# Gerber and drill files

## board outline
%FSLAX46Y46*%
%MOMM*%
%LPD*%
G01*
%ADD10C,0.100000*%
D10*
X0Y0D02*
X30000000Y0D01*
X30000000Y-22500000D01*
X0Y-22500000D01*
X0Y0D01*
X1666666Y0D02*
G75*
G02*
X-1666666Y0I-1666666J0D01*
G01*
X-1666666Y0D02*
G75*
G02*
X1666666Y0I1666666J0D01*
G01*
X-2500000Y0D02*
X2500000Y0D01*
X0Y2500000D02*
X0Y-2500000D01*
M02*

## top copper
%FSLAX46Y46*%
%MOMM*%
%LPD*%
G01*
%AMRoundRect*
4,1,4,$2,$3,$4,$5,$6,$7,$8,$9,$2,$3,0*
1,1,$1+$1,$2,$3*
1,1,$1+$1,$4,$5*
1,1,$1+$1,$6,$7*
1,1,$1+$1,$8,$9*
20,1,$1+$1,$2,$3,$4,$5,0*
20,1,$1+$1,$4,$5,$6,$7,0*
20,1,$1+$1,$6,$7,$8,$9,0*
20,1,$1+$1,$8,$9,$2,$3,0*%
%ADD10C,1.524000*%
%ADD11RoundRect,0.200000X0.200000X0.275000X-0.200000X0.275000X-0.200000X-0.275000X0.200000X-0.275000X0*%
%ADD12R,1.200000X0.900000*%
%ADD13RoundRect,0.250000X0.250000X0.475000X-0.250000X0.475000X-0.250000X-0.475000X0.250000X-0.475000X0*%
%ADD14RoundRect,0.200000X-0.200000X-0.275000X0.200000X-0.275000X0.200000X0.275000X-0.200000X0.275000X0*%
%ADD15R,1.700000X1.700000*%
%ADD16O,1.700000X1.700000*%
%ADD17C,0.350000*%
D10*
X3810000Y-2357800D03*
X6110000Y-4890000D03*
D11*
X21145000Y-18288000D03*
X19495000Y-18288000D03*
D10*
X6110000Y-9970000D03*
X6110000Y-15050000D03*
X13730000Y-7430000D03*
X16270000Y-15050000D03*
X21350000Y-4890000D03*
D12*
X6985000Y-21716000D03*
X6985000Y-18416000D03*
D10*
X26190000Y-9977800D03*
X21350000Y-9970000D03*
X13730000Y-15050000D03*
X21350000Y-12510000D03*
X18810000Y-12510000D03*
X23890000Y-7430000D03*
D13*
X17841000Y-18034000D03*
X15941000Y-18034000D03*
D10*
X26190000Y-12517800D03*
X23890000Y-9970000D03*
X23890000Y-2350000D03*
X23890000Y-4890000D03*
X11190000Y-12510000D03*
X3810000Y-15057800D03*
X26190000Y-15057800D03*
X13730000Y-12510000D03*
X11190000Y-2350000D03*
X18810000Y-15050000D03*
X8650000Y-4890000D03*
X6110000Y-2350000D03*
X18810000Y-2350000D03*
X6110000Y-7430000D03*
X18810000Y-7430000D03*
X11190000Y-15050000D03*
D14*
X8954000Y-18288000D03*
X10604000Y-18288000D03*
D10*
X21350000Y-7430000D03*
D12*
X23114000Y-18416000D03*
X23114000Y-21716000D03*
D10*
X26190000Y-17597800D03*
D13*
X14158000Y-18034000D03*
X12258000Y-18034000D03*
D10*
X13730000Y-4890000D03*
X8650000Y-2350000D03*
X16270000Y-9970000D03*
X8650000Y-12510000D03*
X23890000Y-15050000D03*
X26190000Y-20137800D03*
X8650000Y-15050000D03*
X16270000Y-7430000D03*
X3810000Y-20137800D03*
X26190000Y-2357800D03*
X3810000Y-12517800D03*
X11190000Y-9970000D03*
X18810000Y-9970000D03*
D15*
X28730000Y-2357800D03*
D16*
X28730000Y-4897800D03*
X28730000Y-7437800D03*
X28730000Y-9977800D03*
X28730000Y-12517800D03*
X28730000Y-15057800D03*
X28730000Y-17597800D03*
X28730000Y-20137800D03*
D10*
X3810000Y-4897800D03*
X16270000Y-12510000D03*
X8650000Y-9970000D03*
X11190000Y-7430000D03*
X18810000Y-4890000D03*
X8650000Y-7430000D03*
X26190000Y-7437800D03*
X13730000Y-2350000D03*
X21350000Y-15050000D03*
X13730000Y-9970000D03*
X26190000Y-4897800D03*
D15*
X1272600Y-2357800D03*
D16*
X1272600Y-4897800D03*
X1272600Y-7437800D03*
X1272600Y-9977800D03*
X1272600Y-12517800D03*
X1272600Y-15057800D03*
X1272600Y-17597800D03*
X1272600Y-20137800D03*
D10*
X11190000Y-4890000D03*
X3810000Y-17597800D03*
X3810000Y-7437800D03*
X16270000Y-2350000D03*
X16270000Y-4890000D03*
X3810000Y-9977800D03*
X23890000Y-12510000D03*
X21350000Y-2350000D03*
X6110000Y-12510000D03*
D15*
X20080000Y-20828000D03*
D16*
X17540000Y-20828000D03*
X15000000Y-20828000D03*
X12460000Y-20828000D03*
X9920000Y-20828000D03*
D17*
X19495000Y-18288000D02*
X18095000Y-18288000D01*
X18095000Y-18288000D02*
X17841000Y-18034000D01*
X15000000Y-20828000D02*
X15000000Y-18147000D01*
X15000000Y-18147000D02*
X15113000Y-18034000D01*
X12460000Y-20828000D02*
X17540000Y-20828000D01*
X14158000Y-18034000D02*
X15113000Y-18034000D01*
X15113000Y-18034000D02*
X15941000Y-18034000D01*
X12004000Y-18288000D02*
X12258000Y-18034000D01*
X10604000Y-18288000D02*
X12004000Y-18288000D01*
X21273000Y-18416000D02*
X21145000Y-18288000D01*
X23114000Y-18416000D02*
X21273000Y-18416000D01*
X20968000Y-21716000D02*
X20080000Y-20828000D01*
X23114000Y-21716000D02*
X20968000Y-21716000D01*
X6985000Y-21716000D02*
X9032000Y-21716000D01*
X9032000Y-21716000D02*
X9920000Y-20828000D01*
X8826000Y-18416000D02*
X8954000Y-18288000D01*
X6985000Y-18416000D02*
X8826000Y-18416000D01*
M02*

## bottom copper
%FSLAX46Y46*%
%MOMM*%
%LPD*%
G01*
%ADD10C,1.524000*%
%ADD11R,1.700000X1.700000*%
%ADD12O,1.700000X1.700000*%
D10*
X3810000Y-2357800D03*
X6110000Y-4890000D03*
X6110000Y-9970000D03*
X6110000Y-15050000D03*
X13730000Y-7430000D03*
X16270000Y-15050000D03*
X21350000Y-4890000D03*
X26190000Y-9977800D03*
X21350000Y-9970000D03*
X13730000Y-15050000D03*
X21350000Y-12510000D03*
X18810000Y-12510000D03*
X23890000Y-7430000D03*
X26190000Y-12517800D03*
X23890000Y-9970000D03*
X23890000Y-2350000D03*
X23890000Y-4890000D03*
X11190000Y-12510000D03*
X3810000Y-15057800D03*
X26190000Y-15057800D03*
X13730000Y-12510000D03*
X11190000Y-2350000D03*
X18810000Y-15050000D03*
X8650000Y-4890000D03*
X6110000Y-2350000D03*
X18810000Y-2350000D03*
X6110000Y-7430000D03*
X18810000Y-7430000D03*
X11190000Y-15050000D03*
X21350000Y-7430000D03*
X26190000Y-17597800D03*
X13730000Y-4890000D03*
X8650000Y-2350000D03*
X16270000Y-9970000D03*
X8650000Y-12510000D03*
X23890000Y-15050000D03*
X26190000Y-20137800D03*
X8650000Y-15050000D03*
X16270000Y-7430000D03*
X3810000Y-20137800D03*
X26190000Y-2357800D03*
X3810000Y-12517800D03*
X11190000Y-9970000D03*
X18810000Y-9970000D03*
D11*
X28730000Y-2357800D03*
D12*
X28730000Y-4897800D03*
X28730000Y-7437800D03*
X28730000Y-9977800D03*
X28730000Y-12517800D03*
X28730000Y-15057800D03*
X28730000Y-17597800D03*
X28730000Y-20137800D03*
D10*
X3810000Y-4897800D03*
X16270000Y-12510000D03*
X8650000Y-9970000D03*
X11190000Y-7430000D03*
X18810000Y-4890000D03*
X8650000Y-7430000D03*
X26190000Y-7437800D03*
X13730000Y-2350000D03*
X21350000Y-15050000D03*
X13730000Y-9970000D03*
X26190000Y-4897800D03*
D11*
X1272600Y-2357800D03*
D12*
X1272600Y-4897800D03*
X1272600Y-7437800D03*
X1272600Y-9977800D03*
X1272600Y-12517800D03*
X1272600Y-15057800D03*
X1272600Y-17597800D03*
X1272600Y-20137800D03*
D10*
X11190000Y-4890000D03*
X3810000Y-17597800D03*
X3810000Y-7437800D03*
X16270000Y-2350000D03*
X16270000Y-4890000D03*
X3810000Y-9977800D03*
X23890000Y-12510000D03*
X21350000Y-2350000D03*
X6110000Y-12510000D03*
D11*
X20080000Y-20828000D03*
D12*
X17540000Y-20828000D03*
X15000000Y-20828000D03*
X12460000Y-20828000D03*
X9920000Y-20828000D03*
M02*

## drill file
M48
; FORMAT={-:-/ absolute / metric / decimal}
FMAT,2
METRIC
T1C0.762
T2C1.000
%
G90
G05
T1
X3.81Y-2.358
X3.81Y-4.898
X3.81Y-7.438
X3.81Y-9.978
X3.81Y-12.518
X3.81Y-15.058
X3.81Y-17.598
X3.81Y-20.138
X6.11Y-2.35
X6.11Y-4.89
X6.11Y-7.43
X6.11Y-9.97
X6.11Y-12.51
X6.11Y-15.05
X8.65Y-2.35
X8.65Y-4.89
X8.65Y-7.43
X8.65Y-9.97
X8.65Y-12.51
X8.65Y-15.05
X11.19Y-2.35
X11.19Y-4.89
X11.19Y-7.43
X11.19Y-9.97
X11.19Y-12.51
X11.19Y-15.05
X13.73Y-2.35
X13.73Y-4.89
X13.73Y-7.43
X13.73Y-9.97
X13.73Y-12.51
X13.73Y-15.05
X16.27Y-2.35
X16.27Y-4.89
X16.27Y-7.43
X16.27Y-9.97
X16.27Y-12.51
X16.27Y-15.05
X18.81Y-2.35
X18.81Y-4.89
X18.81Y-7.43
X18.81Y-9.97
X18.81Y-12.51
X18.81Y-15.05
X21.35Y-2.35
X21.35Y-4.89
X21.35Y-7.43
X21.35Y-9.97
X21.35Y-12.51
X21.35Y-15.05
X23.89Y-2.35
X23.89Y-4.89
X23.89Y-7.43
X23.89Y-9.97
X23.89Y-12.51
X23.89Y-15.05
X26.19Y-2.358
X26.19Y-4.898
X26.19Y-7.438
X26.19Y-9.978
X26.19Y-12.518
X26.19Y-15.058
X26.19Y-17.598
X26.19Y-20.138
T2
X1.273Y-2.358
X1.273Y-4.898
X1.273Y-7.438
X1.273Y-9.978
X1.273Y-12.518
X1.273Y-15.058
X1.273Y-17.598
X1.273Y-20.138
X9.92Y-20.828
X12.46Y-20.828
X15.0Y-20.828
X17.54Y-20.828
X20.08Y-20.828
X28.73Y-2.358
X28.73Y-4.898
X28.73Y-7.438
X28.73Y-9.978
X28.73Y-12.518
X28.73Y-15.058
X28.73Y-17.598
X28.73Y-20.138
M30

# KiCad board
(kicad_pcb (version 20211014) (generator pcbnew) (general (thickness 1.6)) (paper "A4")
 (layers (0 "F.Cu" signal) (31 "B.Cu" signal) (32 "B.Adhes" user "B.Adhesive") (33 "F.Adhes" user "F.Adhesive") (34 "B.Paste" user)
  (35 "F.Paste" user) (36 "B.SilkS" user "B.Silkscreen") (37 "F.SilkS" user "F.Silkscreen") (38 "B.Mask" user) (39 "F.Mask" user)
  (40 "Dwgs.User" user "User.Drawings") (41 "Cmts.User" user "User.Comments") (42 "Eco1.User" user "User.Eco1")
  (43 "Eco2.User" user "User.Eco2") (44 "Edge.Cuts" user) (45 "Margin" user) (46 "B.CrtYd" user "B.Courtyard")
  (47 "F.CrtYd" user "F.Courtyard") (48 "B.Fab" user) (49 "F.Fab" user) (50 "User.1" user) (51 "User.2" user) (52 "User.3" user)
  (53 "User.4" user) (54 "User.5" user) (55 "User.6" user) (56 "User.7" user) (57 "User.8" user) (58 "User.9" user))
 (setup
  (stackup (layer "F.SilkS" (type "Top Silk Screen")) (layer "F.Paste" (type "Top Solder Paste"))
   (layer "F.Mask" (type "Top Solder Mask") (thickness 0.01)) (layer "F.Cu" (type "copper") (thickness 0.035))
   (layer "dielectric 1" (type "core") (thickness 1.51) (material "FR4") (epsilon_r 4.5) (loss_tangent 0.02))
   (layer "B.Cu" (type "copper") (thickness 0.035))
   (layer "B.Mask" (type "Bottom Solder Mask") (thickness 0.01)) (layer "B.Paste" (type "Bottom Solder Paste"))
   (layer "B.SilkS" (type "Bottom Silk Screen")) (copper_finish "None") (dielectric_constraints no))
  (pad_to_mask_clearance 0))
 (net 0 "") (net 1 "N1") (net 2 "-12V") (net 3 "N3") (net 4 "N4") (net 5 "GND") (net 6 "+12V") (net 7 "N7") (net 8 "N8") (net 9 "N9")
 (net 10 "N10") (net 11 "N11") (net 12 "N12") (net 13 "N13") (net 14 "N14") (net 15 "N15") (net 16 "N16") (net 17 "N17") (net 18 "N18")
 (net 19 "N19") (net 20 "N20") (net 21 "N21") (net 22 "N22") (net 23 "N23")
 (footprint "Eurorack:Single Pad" (layer "F.Cu") (at 39.75 2.3578)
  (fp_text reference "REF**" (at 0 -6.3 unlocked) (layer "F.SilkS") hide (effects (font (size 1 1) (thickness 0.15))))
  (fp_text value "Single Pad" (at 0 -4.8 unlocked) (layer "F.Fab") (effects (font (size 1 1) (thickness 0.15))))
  (pad "1" thru_hole circle (at -35.94 0) (size 1.524 1.524) (drill 0.762) (layers *.Cu *.Mask)))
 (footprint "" (layer "F.Cu") (at 6.11 4.89)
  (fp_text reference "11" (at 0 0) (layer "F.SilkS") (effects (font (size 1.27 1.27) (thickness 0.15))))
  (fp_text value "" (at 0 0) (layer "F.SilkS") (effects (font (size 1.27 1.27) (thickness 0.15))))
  (pad "1" thru_hole circle (at 0 0) (size 1.524 1.524) (drill 0.762) (layers *.Cu *.Mask)))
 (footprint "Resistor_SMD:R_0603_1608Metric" (layer "F.Cu") (at 20.32 18.288 180)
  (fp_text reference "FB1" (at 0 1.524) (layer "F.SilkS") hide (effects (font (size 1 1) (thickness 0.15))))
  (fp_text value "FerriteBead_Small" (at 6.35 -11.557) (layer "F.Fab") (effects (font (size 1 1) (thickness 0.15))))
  (pad "1" smd roundrect (at -0.825 0 180) (size 0.8 0.95) (layers "F.Cu" "F.Paste" "F.Mask") (roundrect_rratio 0.25) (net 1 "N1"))
  (pad "2" smd roundrect (at 0.825 0 180) (size 0.8 0.95) (layers "F.Cu" "F.Paste" "F.Mask") (roundrect_rratio 0.25) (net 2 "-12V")))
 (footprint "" (layer "F.Cu") (at 6.11 9.97)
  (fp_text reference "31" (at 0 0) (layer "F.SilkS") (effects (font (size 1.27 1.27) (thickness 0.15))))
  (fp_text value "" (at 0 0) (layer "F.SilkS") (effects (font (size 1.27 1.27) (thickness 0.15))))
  (pad "1" thru_hole circle (at 0 0) (size 1.524 1.524) (drill 0.762) (layers *.Cu *.Mask)))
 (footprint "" (layer "F.Cu") (at 6.11 15.05)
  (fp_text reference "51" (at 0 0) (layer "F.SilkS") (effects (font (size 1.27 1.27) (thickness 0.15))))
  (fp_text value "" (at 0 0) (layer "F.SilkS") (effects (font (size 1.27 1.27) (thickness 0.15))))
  (pad "1" thru_hole circle (at 0 0) (size 1.524 1.524) (drill 0.762) (layers *.Cu *.Mask)))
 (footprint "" (layer "F.Cu") (at 13.73 7.43)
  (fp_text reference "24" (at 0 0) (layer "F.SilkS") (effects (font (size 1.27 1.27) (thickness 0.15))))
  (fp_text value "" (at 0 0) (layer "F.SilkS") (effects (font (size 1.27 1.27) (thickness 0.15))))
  (pad "1" thru_hole circle (at 0 0) (size 1.524 1.524) (drill 0.762) (layers *.Cu *.Mask)))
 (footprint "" (layer "F.Cu") (at 16.27 15.05)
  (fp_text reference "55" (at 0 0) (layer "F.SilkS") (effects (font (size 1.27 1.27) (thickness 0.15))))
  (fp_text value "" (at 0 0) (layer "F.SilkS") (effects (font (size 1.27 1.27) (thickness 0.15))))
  (pad "1" thru_hole circle (at 0 0) (size 1.524 1.524) (drill 0.762) (layers *.Cu *.Mask)))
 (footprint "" (layer "F.Cu") (at 21.35 4.89)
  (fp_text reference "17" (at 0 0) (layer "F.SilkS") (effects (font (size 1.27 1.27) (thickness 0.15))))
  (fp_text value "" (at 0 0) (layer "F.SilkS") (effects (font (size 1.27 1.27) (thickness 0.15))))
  (pad "1" thru_hole circle (at 0 0) (size 1.524 1.524) (drill 0.762) (layers *.Cu *.Mask)))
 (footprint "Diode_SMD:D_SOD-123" (layer "F.Cu") (at 6.985 20.066 90)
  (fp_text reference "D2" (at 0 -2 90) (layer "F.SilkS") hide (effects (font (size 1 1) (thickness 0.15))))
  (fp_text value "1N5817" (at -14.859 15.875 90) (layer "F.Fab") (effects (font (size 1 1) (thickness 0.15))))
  (pad "1" smd rect (at -1.65 0 90) (size 0.9 1.2) (layers "F.Cu" "F.Paste" "F.Mask") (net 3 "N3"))
  (pad "2" smd rect (at 1.65 0 90) (size 0.9 1.2) (layers "F.Cu" "F.Paste" "F.Mask") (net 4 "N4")))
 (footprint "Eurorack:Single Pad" (layer "F.Cu") (at 61.94 9.9778)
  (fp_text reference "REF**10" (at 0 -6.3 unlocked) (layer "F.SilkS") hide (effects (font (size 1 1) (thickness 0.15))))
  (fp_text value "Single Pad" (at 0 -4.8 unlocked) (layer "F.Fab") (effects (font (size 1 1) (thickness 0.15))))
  (pad "1" thru_hole circle (at -35.75 0) (size 1.524 1.524) (drill 0.762) (layers *.Cu *.Mask)))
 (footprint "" (layer "F.Cu") (at 21.35 9.97)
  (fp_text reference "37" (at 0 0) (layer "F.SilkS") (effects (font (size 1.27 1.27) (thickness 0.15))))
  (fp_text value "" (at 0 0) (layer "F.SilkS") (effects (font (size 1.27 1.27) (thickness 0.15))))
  (pad "1" thru_hole circle (at 0 0) (size 1.524 1.524) (drill 0.762) (layers *.Cu *.Mask)))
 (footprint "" (layer "F.Cu") (at 13.73 15.05)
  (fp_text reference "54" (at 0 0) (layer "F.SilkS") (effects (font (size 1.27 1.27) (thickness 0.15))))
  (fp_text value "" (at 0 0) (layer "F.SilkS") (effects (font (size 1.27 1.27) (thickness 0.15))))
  (pad "1" thru_hole circle (at 0 0) (size 1.524 1.524) (drill 0.762) (layers *.Cu *.Mask)))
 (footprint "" (layer "F.Cu") (at 21.35 12.51)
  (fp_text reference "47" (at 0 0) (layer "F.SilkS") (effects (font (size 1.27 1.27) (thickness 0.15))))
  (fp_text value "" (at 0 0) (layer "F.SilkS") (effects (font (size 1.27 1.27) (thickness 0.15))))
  (pad "1" thru_hole circle (at 0 0) (size 1.524 1.524) (drill 0.762) (layers *.Cu *.Mask)))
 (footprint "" (layer "F.Cu") (at 18.81 12.51)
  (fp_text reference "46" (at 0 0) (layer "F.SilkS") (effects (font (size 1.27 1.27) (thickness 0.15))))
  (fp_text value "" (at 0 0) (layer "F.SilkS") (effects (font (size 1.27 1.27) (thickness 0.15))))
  (pad "1" thru_hole circle (at 0 0) (size 1.524 1.524) (drill 0.762) (layers *.Cu *.Mask)))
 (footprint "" (layer "F.Cu") (at 23.89 7.43)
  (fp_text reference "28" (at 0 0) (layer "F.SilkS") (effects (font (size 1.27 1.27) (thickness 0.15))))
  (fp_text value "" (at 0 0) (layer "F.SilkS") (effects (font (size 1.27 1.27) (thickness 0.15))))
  (pad "1" thru_hole circle (at 0 0) (size 1.524 1.524) (drill 0.762) (layers *.Cu *.Mask)))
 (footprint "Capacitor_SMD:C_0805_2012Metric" (layer "F.Cu") (at 16.891 18.034 180)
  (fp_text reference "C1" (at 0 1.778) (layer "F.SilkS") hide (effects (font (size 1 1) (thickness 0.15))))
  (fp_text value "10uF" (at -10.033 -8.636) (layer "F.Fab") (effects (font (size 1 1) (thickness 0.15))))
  (pad "1" smd roundrect (at -0.95 0 180) (size 1 1.45) (layers "F.Cu" "F.Paste" "F.Mask") (roundrect_rratio 0.25) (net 2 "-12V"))
  (pad "2" smd roundrect (at 0.95 0 180) (size 1 1.45) (layers "F.Cu" "F.Paste" "F.Mask") (roundrect_rratio 0.25) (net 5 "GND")))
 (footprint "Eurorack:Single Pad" (layer "F.Cu") (at 61.94 12.5178)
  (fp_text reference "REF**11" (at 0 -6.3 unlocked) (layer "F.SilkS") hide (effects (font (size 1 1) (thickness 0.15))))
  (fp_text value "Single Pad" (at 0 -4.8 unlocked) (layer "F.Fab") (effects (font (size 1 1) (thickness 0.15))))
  (pad "1" thru_hole circle (at -35.75 0) (size 1.524 1.524) (drill 0.762) (layers *.Cu *.Mask)))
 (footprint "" (layer "F.Cu") (at 23.89 9.97)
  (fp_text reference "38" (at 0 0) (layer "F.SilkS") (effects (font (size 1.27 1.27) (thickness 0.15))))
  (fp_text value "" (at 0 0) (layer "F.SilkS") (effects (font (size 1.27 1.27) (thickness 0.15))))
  (pad "1" thru_hole circle (at 0 0) (size 1.524 1.524) (drill 0.762) (layers *.Cu *.Mask)))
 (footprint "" (layer "F.Cu") (at 23.89 2.35)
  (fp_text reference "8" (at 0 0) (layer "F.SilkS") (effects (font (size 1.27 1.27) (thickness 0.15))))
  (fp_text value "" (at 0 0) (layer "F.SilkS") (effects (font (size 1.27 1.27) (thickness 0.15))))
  (pad "1" thru_hole circle (at 0 0) (size 1.524 1.524) (drill 0.762) (layers *.Cu *.Mask)))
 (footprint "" (layer "F.Cu") (at 23.89 4.89)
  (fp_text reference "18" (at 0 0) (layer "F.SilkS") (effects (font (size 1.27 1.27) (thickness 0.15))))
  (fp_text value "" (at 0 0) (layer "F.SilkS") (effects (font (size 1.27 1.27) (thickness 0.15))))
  (pad "1" thru_hole circle (at 0 0) (size 1.524 1.524) (drill 0.762) (layers *.Cu *.Mask)))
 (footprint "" (layer "F.Cu") (at 11.19 12.51)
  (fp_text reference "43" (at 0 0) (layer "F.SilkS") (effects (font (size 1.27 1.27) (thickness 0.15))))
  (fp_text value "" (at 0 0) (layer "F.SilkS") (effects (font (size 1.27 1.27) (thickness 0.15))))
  (pad "1" thru_hole circle (at 0 0) (size 1.524 1.524) (drill 0.762) (layers *.Cu *.Mask)))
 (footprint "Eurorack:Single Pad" (layer "F.Cu") (at 39.75 15.0578)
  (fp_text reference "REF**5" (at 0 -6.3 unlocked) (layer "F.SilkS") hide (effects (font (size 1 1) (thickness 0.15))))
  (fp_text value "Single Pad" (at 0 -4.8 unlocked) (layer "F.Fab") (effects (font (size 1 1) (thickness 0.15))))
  (pad "1" thru_hole circle (at -35.94 0) (size 1.524 1.524) (drill 0.762) (layers *.Cu *.Mask)))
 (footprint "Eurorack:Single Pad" (layer "F.Cu") (at 61.94 15.0578)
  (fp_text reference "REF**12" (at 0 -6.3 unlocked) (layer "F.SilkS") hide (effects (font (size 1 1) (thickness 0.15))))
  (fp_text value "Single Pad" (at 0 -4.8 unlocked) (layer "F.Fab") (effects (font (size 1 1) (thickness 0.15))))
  (pad "1" thru_hole circle (at -35.75 0) (size 1.524 1.524) (drill 0.762) (layers *.Cu *.Mask)))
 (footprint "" (layer "F.Cu") (at 13.73 12.51)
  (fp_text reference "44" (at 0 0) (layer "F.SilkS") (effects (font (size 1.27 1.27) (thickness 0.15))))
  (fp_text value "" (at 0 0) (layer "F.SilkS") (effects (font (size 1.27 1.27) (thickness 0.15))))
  (pad "1" thru_hole circle (at 0 0) (size 1.524 1.524) (drill 0.762) (layers *.Cu *.Mask)))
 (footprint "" (layer "F.Cu") (at 11.19 2.35)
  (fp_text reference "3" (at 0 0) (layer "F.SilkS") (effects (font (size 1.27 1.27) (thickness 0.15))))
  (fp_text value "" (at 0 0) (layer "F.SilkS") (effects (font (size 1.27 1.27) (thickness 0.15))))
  (pad "1" thru_hole circle (at 0 0) (size 1.524 1.524) (drill 0.762) (layers *.Cu *.Mask)))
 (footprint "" (layer "F.Cu") (at 18.81 15.05)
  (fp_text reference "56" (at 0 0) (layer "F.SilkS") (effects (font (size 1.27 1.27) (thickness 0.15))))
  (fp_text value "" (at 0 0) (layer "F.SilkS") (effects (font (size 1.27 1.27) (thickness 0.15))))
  (pad "1" thru_hole circle (at 0 0) (size 1.524 1.524) (drill 0.762) (layers *.Cu *.Mask)))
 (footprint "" (layer "F.Cu") (at 8.65 4.89)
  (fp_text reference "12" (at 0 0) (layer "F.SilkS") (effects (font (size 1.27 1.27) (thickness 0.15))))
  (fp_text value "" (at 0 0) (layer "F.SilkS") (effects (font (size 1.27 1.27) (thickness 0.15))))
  (pad "1" thru_hole circle (at 0 0) (size 1.524 1.524) (drill 0.762) (layers *.Cu *.Mask)))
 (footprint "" (layer "F.Cu") (at 6.11 2.35)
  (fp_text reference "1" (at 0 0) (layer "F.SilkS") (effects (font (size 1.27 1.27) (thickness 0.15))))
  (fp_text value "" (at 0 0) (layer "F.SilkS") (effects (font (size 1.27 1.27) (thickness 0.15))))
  (pad "1" thru_hole circle (at 0 0) (size 1.524 1.524) (drill 0.762) (layers *.Cu *.Mask)))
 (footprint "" (layer "F.Cu") (at 18.81 2.35)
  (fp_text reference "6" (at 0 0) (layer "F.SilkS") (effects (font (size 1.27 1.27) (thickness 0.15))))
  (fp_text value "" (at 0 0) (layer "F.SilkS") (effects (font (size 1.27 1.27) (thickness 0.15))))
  (pad "1" thru_hole circle (at 0 0) (size 1.524 1.524) (drill 0.762) (layers *.Cu *.Mask)))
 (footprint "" (layer "F.Cu") (at 6.11 7.43)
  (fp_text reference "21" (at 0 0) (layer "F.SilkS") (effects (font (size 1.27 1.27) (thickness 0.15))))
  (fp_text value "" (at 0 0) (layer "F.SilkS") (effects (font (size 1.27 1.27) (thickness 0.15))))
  (pad "1" thru_hole circle (at 0 0) (size 1.524 1.524) (drill 0.762) (layers *.Cu *.Mask)))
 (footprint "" (layer "F.Cu") (at 18.81 7.43)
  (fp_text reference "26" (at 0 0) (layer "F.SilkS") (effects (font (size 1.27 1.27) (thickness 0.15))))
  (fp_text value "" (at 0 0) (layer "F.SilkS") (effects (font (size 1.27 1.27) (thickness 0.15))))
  (pad "1" thru_hole circle (at 0 0) (size 1.524 1.524) (drill 0.762) (layers *.Cu *.Mask)))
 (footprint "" (layer "F.Cu") (at 11.19 15.05)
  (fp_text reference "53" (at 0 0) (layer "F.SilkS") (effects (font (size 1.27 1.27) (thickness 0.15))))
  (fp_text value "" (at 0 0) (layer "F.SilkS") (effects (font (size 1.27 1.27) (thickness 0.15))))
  (pad "1" thru_hole circle (at 0 0) (size 1.524 1.524) (drill 0.762) (layers *.Cu *.Mask)))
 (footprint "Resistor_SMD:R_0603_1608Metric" (layer "F.Cu") (at 9.779 18.288)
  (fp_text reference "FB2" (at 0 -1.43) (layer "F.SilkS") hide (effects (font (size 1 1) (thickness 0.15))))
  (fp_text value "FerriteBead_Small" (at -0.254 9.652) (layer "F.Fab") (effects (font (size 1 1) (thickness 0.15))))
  (pad "1" smd roundrect (at -0.825 0) (size 0.8 0.95) (layers "F.Cu" "F.Paste" "F.Mask") (roundrect_rratio 0.25) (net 4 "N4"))
  (pad "2" smd roundrect (at 0.825 0) (size 0.8 0.95) (layers "F.Cu" "F.Paste" "F.Mask") (roundrect_rratio 0.25) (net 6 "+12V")))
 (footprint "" (layer "F.Cu") (at 21.35 7.43)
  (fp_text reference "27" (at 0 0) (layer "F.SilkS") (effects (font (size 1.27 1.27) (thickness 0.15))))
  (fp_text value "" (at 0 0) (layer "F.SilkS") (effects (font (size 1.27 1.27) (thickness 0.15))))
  (pad "1" thru_hole circle (at 0 0) (size 1.524 1.524) (drill 0.762) (layers *.Cu *.Mask)))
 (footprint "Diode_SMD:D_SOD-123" (layer "F.Cu") (at 23.114 20.066 -90)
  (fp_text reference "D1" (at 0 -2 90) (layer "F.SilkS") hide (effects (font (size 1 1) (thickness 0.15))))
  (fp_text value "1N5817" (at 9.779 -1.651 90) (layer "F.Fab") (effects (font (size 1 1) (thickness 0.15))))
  (pad "1" smd rect (at -1.65 0 270) (size 0.9 1.2) (layers "F.Cu" "F.Paste" "F.Mask") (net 1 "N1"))
  (pad "2" smd rect (at 1.65 0 270) (size 0.9 1.2) (layers "F.Cu" "F.Paste" "F.Mask") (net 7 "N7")))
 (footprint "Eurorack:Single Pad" (layer "F.Cu") (at 61.94 17.5978)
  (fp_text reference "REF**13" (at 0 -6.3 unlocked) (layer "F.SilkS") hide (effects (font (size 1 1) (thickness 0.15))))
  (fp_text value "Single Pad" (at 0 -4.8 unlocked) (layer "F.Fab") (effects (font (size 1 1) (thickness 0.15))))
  (pad "1" thru_hole circle (at -35.75 0) (size 1.524 1.524) (drill 0.762) (layers *.Cu *.Mask)))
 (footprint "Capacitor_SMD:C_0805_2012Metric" (layer "F.Cu") (at 13.208 18.034 180)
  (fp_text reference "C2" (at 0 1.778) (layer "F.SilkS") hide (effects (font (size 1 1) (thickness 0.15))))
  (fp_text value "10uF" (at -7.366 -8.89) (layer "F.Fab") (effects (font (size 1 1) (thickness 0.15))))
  (pad "1" smd roundrect (at -0.95 0 180) (size 1 1.45) (layers "F.Cu" "F.Paste" "F.Mask") (roundrect_rratio 0.25) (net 5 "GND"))
  (pad "2" smd roundrect (at 0.95 0 180) (size 1 1.45) (layers "F.Cu" "F.Paste" "F.Mask") (roundrect_rratio 0.25) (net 6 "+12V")))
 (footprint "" (layer "F.Cu") (at 13.73 4.89)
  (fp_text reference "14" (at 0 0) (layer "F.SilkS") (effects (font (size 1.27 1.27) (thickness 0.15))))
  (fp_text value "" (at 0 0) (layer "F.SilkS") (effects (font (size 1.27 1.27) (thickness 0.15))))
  (pad "1" thru_hole circle (at 0 0) (size 1.524 1.524) (drill 0.762) (layers *.Cu *.Mask)))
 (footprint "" (layer "F.Cu") (at 8.65 2.35)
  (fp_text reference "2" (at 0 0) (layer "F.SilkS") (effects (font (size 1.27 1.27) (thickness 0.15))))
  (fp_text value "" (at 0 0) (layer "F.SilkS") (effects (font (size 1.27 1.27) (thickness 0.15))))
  (pad "1" thru_hole circle (at 0 0) (size 1.524 1.524) (drill 0.762) (layers *.Cu *.Mask)))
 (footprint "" (layer "F.Cu") (at 16.27 9.97)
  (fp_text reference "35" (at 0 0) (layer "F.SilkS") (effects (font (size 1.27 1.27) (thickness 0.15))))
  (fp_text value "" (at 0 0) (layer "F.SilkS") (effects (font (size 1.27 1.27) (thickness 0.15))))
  (pad "1" thru_hole circle (at 0 0) (size 1.524 1.524) (drill 0.762) (layers *.Cu *.Mask)))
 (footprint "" (layer "F.Cu") (at 8.65 12.51)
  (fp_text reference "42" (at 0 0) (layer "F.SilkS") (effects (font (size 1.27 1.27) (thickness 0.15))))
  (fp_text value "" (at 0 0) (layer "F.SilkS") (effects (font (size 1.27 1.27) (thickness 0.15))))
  (pad "1" thru_hole circle (at 0 0) (size 1.524 1.524) (drill 0.762) (layers *.Cu *.Mask)))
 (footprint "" (layer "F.Cu") (at 23.89 15.05)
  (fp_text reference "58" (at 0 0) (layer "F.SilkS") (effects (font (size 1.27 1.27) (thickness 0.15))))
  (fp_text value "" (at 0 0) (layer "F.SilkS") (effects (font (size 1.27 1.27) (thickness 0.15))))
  (pad "1" thru_hole circle (at 0 0) (size 1.524 1.524) (drill 0.762) (layers *.Cu *.Mask)))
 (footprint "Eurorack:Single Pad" (layer "F.Cu") (at 61.94 20.1378)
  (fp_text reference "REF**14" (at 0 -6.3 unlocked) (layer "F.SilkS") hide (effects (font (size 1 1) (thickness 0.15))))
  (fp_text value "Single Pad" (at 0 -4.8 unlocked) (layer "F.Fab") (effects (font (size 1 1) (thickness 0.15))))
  (pad "1" thru_hole circle (at -35.75 0) (size 1.524 1.524) (drill 0.762) (layers *.Cu *.Mask)))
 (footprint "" (layer "F.Cu") (at 8.65 15.05)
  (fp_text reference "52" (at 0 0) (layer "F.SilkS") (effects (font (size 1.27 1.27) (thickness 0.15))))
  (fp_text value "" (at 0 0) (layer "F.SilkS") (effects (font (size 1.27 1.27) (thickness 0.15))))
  (pad "1" thru_hole circle (at 0 0) (size 1.524 1.524) (drill 0.762) (layers *.Cu *.Mask)))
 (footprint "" (layer "F.Cu") (at 16.27 7.43)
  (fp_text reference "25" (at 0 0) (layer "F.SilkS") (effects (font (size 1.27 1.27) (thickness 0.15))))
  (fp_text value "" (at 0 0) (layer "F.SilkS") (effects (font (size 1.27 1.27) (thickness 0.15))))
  (pad "1" thru_hole circle (at 0 0) (size 1.524 1.524) (drill 0.762) (layers *.Cu *.Mask)))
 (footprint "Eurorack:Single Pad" (layer "F.Cu") (at 39.75 20.1378)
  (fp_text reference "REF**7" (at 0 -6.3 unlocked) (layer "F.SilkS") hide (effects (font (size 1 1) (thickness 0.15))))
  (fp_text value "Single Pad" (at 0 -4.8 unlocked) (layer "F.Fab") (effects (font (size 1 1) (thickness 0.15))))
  (pad "1" thru_hole circle (at -35.94 0) (size 1.524 1.524) (drill 0.762) (layers *.Cu *.Mask)))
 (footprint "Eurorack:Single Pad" (layer "F.Cu") (at 61.94 2.3578)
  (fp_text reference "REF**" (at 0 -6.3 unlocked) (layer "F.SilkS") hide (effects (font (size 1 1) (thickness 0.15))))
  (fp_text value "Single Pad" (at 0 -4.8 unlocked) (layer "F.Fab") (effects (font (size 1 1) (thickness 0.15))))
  (pad "1" thru_hole circle (at -35.75 0) (size 1.524 1.524) (drill 0.762) (layers *.Cu *.Mask)))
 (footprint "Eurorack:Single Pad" (layer "F.Cu") (at 39.75 12.5178)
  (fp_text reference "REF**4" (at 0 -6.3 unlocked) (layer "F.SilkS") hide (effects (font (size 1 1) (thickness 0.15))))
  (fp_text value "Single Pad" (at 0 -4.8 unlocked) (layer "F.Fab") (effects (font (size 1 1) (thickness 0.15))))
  (pad "1" thru_hole circle (at -35.94 0) (size 1.524 1.524) (drill 0.762) (layers *.Cu *.Mask)))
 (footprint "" (layer "F.Cu") (at 11.19 9.97)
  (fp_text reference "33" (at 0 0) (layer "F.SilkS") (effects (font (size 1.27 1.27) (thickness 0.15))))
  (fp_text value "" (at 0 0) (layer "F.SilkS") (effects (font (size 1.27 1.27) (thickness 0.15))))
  (pad "1" thru_hole circle (at 0 0) (size 1.524 1.524) (drill 0.762) (layers *.Cu *.Mask)))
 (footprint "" (layer "F.Cu") (at 18.81 9.97)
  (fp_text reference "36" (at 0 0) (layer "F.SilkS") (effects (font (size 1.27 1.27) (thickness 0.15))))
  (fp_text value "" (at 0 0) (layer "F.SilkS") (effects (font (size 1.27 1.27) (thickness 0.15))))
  (pad "1" thru_hole circle (at 0 0) (size 1.524 1.524) (drill 0.762) (layers *.Cu *.Mask)))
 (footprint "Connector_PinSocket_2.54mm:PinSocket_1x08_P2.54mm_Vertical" (layer "F.Cu") (at 28.73 2.3578)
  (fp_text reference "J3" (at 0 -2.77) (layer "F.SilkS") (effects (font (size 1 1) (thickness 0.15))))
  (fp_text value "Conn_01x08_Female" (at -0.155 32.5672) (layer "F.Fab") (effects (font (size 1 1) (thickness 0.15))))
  (pad "1" thru_hole rect (at 0 0) (size 1.7 1.7) (drill 1) (layers *.Cu *.Mask) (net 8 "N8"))
  (pad "2" thru_hole oval (at 0 2.54) (size 1.7 1.7) (drill 1) (layers *.Cu *.Mask) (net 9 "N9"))
  (pad "3" thru_hole oval (at 0 5.08) (size 1.7 1.7) (drill 1) (layers *.Cu *.Mask) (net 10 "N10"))
  (pad "4" thru_hole oval (at 0 7.62) (size 1.7 1.7) (drill 1) (layers *.Cu *.Mask) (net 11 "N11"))
  (pad "5" thru_hole oval (at 0 10.16) (size 1.7 1.7) (drill 1) (layers *.Cu *.Mask) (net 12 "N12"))
  (pad "6" thru_hole oval (at 0 12.7) (size 1.7 1.7) (drill 1) (layers *.Cu *.Mask) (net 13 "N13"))
  (pad "7" thru_hole oval (at 0 15.24) (size 1.7 1.7) (drill 1) (layers *.Cu *.Mask) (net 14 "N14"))
  (pad "8" thru_hole oval (at 0 17.78) (size 1.7 1.7) (drill 1) (layers *.Cu *.Mask) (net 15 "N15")))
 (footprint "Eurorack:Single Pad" (layer "F.Cu") (at 39.75 4.8978)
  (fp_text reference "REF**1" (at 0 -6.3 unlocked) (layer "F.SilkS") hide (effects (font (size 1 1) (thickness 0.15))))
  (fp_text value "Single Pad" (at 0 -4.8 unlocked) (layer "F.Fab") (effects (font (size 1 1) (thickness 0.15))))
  (pad "1" thru_hole circle (at -35.94 0) (size 1.524 1.524) (drill 0.762) (layers *.Cu *.Mask)))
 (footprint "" (layer "F.Cu") (at 16.27 12.51)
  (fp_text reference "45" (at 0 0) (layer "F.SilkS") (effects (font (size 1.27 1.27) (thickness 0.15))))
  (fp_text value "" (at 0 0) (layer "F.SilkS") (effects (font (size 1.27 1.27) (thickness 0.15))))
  (pad "1" thru_hole circle (at 0 0) (size 1.524 1.524) (drill 0.762) (layers *.Cu *.Mask)))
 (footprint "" (layer "F.Cu") (at 8.65 9.97)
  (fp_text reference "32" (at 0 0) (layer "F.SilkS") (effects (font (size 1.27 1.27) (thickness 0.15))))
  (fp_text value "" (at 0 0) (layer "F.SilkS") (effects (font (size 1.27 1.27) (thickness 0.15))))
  (pad "1" thru_hole circle (at 0 0) (size 1.524 1.524) (drill 0.762) (layers *.Cu *.Mask)))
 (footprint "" (layer "F.Cu") (at 11.19 7.43)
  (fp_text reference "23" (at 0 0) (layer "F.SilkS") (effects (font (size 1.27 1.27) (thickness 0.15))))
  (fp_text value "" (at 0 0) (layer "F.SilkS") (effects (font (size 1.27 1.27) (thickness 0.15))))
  (pad "1" thru_hole circle (at 0 0) (size 1.524 1.524) (drill 0.762) (layers *.Cu *.Mask)))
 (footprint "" (layer "F.Cu") (at 18.81 4.89)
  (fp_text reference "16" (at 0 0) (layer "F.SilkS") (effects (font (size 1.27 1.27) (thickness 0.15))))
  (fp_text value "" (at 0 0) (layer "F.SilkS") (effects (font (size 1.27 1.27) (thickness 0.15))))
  (pad "1" thru_hole circle (at 0 0) (size 1.524 1.524) (drill 0.762) (layers *.Cu *.Mask)))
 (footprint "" (layer "F.Cu") (at 8.65 7.43)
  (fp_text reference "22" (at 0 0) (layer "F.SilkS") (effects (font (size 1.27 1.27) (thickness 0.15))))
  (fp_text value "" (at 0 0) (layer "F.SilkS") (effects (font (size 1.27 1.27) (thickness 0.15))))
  (pad "1" thru_hole circle (at 0 0) (size 1.524 1.524) (drill 0.762) (layers *.Cu *.Mask)))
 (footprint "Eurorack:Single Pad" (layer "F.Cu") (at 61.94 7.4378)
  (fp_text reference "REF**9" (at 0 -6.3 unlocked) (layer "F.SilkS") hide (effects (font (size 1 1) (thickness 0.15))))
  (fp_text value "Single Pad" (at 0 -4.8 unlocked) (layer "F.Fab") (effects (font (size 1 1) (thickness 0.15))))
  (pad "1" thru_hole circle (at -35.75 0) (size 1.524 1.524) (drill 0.762) (layers *.Cu *.Mask)))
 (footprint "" (layer "F.Cu") (at 13.73 2.35)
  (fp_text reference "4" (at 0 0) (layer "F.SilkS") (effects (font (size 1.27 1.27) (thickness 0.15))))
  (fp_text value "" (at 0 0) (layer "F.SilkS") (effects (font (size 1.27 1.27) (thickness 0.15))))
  (pad "1" thru_hole circle (at 0 0) (size 1.524 1.524) (drill 0.762) (layers *.Cu *.Mask)))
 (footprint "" (layer "F.Cu") (at 21.35 15.05)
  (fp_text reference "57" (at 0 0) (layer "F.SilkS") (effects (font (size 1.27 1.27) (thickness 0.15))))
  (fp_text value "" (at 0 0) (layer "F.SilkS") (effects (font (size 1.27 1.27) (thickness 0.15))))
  (pad "1" thru_hole circle (at 0 0) (size 1.524 1.524) (drill 0.762) (layers *.Cu *.Mask)))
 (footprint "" (layer "F.Cu") (at 13.73 9.97)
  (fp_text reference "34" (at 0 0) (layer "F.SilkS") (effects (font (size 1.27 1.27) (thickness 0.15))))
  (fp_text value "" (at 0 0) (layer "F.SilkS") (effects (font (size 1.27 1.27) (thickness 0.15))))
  (pad "1" thru_hole circle (at 0 0) (size 1.524 1.524) (drill 0.762) (layers *.Cu *.Mask)))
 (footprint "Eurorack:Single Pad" (layer "F.Cu") (at 61.94 4.8978)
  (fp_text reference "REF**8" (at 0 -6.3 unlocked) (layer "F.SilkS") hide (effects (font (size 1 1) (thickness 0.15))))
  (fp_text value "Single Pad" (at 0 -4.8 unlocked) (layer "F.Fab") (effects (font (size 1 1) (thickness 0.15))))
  (pad "1" thru_hole circle (at -35.75 0) (size 1.524 1.524) (drill 0.762) (layers *.Cu *.Mask)))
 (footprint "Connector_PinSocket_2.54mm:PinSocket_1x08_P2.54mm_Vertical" (layer "F.Cu") (at 1.2726 2.3578)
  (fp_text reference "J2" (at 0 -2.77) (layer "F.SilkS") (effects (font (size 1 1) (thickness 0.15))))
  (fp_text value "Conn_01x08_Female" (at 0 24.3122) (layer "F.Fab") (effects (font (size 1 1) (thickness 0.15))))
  (pad "1" thru_hole rect (at 0 0) (size 1.7 1.7) (drill 1) (layers *.Cu *.Mask) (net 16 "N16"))
  (pad "2" thru_hole oval (at 0 2.54) (size 1.7 1.7) (drill 1) (layers *.Cu *.Mask) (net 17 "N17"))
  (pad "3" thru_hole oval (at 0 5.08) (size 1.7 1.7) (drill 1) (layers *.Cu *.Mask) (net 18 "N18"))
  (pad "4" thru_hole oval (at 0 7.62) (size 1.7 1.7) (drill 1) (layers *.Cu *.Mask) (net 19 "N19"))
  (pad "5" thru_hole oval (at 0 10.16) (size 1.7 1.7) (drill 1) (layers *.Cu *.Mask) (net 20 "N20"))
  (pad "6" thru_hole oval (at 0 12.7) (size 1.7 1.7) (drill 1) (layers *.Cu *.Mask) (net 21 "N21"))
  (pad "7" thru_hole oval (at 0 15.24) (size 1.7 1.7) (drill 1) (layers *.Cu *.Mask) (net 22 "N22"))
  (pad "8" thru_hole oval (at 0 17.78) (size 1.7 1.7) (drill 1) (layers *.Cu *.Mask) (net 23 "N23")))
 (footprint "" (layer "F.Cu") (at 11.19 4.89)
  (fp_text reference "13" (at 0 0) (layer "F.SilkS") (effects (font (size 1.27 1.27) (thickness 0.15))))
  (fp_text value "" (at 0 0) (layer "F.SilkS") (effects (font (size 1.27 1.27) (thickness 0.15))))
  (pad "1" thru_hole circle (at 0 0) (size 1.524 1.524) (drill 0.762) (layers *.Cu *.Mask)))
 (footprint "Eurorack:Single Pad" (layer "F.Cu") (at 39.75 17.5978)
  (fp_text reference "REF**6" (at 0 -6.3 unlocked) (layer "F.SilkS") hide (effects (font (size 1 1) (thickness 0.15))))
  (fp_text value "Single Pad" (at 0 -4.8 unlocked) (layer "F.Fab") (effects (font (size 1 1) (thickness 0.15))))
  (pad "1" thru_hole circle (at -35.94 0) (size 1.524 1.524) (drill 0.762) (layers *.Cu *.Mask)))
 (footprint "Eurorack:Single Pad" (layer "F.Cu") (at 39.75 7.4378)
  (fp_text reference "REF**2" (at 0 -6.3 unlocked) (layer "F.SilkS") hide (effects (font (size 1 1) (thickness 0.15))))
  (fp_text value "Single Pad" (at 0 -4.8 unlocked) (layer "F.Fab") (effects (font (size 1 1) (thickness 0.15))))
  (pad "1" thru_hole circle (at -35.94 0) (size 1.524 1.524) (drill 0.762) (layers *.Cu *.Mask)))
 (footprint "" (layer "F.Cu") (at 16.27 2.35)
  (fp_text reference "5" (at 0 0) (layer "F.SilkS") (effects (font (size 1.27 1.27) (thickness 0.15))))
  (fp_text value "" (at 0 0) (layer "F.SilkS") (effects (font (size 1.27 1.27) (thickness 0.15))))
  (pad "1" thru_hole circle (at 0 0) (size 1.524 1.524) (drill 0.762) (layers *.Cu *.Mask)))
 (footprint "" (layer "F.Cu") (at 16.27 4.89)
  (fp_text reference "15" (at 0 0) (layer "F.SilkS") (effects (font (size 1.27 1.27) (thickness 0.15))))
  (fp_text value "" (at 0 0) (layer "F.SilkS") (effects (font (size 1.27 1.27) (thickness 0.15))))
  (pad "1" thru_hole circle (at 0 0) (size 1.524 1.524) (drill 0.762) (layers *.Cu *.Mask)))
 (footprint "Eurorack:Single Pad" (layer "F.Cu") (at 39.75 9.9778)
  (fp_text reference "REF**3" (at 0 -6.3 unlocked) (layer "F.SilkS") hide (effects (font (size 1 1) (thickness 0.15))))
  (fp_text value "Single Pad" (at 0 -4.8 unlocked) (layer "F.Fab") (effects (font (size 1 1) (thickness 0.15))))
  (pad "1" thru_hole circle (at -35.94 0) (size 1.524 1.524) (drill 0.762) (layers *.Cu *.Mask)))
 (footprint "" (layer "F.Cu") (at 23.89 12.51)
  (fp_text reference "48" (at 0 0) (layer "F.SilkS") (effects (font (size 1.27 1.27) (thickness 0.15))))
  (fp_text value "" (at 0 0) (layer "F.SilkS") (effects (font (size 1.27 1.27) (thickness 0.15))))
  (pad "1" thru_hole circle (at 0 0) (size 1.524 1.524) (drill 0.762) (layers *.Cu *.Mask)))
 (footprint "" (layer "F.Cu") (at 21.35 2.35)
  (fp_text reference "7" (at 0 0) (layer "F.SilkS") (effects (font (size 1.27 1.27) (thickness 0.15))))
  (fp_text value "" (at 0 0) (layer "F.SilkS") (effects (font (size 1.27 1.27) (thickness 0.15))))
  (pad "1" thru_hole circle (at 0 0) (size 1.524 1.524) (drill 0.762) (layers *.Cu *.Mask)))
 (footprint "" (layer "F.Cu") (at 6.11 12.51)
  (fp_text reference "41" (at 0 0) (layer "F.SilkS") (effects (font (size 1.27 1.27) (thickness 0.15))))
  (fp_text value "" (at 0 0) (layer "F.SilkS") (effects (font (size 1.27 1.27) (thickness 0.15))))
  (pad "1" thru_hole circle (at 0 0) (size 1.524 1.524) (drill 0.762) (layers *.Cu *.Mask)))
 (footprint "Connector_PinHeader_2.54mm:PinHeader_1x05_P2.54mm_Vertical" (layer "B.Cu") (at 20.08 20.828 90)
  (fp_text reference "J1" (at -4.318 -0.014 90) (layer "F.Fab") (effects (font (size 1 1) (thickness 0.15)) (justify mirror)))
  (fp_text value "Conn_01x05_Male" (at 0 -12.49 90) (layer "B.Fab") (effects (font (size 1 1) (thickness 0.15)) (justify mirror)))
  (pad "1" thru_hole rect (at 0 0 90) (size 1.7 1.7) (drill 1) (layers *.Cu *.Mask) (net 7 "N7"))
  (pad "2" thru_hole oval (at 0 -2.54 90) (size 1.7 1.7) (drill 1) (layers *.Cu *.Mask) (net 5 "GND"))
  (pad "3" thru_hole oval (at 0 -5.08 90) (size 1.7 1.7) (drill 1) (layers *.Cu *.Mask) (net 5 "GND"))
  (pad "4" thru_hole oval (at 0 -7.62 90) (size 1.7 1.7) (drill 1) (layers *.Cu *.Mask) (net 5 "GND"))
  (pad "5" thru_hole oval (at 0 -10.16 90) (size 1.7 1.7) (drill 1) (layers *.Cu *.Mask) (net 3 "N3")))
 (gr_rect (start 0 0) (end 30 22.5) (layer "Edge.Cuts") (width 0.1) (fill none))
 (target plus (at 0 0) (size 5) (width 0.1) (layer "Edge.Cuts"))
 (segment (start 19.495 18.288) (end 18.095 18.288) (width 0.35) (layer "F.Cu") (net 2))
 (segment (start 18.095 18.288) (end 17.841 18.034) (width 0.35) (layer "F.Cu") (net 2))
 (segment (start 15 20.828) (end 15 18.147) (width 0.35) (layer "F.Cu") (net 5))
 (segment (start 15 18.147) (end 15.113 18.034) (width 0.35) (layer "F.Cu") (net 5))
 (segment (start 12.46 20.828) (end 17.54 20.828) (width 0.35) (layer "F.Cu") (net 5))
 (segment (start 14.158 18.034) (end 15.113 18.034) (width 0.35) (layer "F.Cu") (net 5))
 (segment (start 15.113 18.034) (end 15.941 18.034) (width 0.35) (layer "F.Cu") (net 5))
 (segment (start 12.004 18.288) (end 12.258 18.034) (width 0.35) (layer "F.Cu") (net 6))
 (segment (start 10.604 18.288) (end 12.004 18.288) (width 0.35) (layer "F.Cu") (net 6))
 (segment (start 21.273 18.416) (end 21.145 18.288) (width 0.35) (layer "F.Cu") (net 1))
 (segment (start 23.114 18.416) (end 21.273 18.416) (width 0.35) (layer "F.Cu") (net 1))
 (segment (start 20.968 21.716) (end 20.08 20.828) (width 0.35) (layer "F.Cu") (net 7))
 (segment (start 23.114 21.716) (end 20.968 21.716) (width 0.35) (layer "F.Cu") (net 7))
 (segment (start 6.985 21.716) (end 9.032 21.716) (width 0.35) (layer "F.Cu") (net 3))
 (segment (start 9.032 21.716) (end 9.92 20.828) (width 0.35) (layer "F.Cu") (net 3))
 (segment (start 8.826 18.416) (end 8.954 18.288) (width 0.35) (layer "F.Cu") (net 4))
 (segment (start 6.985 18.416) (end 8.826 18.416) (width 0.35) (layer "F.Cu") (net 4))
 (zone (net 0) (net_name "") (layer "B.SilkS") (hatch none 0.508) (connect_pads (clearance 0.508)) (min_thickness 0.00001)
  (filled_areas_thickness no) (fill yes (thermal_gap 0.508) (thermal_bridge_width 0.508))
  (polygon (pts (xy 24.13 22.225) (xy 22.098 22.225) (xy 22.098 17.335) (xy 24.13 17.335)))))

